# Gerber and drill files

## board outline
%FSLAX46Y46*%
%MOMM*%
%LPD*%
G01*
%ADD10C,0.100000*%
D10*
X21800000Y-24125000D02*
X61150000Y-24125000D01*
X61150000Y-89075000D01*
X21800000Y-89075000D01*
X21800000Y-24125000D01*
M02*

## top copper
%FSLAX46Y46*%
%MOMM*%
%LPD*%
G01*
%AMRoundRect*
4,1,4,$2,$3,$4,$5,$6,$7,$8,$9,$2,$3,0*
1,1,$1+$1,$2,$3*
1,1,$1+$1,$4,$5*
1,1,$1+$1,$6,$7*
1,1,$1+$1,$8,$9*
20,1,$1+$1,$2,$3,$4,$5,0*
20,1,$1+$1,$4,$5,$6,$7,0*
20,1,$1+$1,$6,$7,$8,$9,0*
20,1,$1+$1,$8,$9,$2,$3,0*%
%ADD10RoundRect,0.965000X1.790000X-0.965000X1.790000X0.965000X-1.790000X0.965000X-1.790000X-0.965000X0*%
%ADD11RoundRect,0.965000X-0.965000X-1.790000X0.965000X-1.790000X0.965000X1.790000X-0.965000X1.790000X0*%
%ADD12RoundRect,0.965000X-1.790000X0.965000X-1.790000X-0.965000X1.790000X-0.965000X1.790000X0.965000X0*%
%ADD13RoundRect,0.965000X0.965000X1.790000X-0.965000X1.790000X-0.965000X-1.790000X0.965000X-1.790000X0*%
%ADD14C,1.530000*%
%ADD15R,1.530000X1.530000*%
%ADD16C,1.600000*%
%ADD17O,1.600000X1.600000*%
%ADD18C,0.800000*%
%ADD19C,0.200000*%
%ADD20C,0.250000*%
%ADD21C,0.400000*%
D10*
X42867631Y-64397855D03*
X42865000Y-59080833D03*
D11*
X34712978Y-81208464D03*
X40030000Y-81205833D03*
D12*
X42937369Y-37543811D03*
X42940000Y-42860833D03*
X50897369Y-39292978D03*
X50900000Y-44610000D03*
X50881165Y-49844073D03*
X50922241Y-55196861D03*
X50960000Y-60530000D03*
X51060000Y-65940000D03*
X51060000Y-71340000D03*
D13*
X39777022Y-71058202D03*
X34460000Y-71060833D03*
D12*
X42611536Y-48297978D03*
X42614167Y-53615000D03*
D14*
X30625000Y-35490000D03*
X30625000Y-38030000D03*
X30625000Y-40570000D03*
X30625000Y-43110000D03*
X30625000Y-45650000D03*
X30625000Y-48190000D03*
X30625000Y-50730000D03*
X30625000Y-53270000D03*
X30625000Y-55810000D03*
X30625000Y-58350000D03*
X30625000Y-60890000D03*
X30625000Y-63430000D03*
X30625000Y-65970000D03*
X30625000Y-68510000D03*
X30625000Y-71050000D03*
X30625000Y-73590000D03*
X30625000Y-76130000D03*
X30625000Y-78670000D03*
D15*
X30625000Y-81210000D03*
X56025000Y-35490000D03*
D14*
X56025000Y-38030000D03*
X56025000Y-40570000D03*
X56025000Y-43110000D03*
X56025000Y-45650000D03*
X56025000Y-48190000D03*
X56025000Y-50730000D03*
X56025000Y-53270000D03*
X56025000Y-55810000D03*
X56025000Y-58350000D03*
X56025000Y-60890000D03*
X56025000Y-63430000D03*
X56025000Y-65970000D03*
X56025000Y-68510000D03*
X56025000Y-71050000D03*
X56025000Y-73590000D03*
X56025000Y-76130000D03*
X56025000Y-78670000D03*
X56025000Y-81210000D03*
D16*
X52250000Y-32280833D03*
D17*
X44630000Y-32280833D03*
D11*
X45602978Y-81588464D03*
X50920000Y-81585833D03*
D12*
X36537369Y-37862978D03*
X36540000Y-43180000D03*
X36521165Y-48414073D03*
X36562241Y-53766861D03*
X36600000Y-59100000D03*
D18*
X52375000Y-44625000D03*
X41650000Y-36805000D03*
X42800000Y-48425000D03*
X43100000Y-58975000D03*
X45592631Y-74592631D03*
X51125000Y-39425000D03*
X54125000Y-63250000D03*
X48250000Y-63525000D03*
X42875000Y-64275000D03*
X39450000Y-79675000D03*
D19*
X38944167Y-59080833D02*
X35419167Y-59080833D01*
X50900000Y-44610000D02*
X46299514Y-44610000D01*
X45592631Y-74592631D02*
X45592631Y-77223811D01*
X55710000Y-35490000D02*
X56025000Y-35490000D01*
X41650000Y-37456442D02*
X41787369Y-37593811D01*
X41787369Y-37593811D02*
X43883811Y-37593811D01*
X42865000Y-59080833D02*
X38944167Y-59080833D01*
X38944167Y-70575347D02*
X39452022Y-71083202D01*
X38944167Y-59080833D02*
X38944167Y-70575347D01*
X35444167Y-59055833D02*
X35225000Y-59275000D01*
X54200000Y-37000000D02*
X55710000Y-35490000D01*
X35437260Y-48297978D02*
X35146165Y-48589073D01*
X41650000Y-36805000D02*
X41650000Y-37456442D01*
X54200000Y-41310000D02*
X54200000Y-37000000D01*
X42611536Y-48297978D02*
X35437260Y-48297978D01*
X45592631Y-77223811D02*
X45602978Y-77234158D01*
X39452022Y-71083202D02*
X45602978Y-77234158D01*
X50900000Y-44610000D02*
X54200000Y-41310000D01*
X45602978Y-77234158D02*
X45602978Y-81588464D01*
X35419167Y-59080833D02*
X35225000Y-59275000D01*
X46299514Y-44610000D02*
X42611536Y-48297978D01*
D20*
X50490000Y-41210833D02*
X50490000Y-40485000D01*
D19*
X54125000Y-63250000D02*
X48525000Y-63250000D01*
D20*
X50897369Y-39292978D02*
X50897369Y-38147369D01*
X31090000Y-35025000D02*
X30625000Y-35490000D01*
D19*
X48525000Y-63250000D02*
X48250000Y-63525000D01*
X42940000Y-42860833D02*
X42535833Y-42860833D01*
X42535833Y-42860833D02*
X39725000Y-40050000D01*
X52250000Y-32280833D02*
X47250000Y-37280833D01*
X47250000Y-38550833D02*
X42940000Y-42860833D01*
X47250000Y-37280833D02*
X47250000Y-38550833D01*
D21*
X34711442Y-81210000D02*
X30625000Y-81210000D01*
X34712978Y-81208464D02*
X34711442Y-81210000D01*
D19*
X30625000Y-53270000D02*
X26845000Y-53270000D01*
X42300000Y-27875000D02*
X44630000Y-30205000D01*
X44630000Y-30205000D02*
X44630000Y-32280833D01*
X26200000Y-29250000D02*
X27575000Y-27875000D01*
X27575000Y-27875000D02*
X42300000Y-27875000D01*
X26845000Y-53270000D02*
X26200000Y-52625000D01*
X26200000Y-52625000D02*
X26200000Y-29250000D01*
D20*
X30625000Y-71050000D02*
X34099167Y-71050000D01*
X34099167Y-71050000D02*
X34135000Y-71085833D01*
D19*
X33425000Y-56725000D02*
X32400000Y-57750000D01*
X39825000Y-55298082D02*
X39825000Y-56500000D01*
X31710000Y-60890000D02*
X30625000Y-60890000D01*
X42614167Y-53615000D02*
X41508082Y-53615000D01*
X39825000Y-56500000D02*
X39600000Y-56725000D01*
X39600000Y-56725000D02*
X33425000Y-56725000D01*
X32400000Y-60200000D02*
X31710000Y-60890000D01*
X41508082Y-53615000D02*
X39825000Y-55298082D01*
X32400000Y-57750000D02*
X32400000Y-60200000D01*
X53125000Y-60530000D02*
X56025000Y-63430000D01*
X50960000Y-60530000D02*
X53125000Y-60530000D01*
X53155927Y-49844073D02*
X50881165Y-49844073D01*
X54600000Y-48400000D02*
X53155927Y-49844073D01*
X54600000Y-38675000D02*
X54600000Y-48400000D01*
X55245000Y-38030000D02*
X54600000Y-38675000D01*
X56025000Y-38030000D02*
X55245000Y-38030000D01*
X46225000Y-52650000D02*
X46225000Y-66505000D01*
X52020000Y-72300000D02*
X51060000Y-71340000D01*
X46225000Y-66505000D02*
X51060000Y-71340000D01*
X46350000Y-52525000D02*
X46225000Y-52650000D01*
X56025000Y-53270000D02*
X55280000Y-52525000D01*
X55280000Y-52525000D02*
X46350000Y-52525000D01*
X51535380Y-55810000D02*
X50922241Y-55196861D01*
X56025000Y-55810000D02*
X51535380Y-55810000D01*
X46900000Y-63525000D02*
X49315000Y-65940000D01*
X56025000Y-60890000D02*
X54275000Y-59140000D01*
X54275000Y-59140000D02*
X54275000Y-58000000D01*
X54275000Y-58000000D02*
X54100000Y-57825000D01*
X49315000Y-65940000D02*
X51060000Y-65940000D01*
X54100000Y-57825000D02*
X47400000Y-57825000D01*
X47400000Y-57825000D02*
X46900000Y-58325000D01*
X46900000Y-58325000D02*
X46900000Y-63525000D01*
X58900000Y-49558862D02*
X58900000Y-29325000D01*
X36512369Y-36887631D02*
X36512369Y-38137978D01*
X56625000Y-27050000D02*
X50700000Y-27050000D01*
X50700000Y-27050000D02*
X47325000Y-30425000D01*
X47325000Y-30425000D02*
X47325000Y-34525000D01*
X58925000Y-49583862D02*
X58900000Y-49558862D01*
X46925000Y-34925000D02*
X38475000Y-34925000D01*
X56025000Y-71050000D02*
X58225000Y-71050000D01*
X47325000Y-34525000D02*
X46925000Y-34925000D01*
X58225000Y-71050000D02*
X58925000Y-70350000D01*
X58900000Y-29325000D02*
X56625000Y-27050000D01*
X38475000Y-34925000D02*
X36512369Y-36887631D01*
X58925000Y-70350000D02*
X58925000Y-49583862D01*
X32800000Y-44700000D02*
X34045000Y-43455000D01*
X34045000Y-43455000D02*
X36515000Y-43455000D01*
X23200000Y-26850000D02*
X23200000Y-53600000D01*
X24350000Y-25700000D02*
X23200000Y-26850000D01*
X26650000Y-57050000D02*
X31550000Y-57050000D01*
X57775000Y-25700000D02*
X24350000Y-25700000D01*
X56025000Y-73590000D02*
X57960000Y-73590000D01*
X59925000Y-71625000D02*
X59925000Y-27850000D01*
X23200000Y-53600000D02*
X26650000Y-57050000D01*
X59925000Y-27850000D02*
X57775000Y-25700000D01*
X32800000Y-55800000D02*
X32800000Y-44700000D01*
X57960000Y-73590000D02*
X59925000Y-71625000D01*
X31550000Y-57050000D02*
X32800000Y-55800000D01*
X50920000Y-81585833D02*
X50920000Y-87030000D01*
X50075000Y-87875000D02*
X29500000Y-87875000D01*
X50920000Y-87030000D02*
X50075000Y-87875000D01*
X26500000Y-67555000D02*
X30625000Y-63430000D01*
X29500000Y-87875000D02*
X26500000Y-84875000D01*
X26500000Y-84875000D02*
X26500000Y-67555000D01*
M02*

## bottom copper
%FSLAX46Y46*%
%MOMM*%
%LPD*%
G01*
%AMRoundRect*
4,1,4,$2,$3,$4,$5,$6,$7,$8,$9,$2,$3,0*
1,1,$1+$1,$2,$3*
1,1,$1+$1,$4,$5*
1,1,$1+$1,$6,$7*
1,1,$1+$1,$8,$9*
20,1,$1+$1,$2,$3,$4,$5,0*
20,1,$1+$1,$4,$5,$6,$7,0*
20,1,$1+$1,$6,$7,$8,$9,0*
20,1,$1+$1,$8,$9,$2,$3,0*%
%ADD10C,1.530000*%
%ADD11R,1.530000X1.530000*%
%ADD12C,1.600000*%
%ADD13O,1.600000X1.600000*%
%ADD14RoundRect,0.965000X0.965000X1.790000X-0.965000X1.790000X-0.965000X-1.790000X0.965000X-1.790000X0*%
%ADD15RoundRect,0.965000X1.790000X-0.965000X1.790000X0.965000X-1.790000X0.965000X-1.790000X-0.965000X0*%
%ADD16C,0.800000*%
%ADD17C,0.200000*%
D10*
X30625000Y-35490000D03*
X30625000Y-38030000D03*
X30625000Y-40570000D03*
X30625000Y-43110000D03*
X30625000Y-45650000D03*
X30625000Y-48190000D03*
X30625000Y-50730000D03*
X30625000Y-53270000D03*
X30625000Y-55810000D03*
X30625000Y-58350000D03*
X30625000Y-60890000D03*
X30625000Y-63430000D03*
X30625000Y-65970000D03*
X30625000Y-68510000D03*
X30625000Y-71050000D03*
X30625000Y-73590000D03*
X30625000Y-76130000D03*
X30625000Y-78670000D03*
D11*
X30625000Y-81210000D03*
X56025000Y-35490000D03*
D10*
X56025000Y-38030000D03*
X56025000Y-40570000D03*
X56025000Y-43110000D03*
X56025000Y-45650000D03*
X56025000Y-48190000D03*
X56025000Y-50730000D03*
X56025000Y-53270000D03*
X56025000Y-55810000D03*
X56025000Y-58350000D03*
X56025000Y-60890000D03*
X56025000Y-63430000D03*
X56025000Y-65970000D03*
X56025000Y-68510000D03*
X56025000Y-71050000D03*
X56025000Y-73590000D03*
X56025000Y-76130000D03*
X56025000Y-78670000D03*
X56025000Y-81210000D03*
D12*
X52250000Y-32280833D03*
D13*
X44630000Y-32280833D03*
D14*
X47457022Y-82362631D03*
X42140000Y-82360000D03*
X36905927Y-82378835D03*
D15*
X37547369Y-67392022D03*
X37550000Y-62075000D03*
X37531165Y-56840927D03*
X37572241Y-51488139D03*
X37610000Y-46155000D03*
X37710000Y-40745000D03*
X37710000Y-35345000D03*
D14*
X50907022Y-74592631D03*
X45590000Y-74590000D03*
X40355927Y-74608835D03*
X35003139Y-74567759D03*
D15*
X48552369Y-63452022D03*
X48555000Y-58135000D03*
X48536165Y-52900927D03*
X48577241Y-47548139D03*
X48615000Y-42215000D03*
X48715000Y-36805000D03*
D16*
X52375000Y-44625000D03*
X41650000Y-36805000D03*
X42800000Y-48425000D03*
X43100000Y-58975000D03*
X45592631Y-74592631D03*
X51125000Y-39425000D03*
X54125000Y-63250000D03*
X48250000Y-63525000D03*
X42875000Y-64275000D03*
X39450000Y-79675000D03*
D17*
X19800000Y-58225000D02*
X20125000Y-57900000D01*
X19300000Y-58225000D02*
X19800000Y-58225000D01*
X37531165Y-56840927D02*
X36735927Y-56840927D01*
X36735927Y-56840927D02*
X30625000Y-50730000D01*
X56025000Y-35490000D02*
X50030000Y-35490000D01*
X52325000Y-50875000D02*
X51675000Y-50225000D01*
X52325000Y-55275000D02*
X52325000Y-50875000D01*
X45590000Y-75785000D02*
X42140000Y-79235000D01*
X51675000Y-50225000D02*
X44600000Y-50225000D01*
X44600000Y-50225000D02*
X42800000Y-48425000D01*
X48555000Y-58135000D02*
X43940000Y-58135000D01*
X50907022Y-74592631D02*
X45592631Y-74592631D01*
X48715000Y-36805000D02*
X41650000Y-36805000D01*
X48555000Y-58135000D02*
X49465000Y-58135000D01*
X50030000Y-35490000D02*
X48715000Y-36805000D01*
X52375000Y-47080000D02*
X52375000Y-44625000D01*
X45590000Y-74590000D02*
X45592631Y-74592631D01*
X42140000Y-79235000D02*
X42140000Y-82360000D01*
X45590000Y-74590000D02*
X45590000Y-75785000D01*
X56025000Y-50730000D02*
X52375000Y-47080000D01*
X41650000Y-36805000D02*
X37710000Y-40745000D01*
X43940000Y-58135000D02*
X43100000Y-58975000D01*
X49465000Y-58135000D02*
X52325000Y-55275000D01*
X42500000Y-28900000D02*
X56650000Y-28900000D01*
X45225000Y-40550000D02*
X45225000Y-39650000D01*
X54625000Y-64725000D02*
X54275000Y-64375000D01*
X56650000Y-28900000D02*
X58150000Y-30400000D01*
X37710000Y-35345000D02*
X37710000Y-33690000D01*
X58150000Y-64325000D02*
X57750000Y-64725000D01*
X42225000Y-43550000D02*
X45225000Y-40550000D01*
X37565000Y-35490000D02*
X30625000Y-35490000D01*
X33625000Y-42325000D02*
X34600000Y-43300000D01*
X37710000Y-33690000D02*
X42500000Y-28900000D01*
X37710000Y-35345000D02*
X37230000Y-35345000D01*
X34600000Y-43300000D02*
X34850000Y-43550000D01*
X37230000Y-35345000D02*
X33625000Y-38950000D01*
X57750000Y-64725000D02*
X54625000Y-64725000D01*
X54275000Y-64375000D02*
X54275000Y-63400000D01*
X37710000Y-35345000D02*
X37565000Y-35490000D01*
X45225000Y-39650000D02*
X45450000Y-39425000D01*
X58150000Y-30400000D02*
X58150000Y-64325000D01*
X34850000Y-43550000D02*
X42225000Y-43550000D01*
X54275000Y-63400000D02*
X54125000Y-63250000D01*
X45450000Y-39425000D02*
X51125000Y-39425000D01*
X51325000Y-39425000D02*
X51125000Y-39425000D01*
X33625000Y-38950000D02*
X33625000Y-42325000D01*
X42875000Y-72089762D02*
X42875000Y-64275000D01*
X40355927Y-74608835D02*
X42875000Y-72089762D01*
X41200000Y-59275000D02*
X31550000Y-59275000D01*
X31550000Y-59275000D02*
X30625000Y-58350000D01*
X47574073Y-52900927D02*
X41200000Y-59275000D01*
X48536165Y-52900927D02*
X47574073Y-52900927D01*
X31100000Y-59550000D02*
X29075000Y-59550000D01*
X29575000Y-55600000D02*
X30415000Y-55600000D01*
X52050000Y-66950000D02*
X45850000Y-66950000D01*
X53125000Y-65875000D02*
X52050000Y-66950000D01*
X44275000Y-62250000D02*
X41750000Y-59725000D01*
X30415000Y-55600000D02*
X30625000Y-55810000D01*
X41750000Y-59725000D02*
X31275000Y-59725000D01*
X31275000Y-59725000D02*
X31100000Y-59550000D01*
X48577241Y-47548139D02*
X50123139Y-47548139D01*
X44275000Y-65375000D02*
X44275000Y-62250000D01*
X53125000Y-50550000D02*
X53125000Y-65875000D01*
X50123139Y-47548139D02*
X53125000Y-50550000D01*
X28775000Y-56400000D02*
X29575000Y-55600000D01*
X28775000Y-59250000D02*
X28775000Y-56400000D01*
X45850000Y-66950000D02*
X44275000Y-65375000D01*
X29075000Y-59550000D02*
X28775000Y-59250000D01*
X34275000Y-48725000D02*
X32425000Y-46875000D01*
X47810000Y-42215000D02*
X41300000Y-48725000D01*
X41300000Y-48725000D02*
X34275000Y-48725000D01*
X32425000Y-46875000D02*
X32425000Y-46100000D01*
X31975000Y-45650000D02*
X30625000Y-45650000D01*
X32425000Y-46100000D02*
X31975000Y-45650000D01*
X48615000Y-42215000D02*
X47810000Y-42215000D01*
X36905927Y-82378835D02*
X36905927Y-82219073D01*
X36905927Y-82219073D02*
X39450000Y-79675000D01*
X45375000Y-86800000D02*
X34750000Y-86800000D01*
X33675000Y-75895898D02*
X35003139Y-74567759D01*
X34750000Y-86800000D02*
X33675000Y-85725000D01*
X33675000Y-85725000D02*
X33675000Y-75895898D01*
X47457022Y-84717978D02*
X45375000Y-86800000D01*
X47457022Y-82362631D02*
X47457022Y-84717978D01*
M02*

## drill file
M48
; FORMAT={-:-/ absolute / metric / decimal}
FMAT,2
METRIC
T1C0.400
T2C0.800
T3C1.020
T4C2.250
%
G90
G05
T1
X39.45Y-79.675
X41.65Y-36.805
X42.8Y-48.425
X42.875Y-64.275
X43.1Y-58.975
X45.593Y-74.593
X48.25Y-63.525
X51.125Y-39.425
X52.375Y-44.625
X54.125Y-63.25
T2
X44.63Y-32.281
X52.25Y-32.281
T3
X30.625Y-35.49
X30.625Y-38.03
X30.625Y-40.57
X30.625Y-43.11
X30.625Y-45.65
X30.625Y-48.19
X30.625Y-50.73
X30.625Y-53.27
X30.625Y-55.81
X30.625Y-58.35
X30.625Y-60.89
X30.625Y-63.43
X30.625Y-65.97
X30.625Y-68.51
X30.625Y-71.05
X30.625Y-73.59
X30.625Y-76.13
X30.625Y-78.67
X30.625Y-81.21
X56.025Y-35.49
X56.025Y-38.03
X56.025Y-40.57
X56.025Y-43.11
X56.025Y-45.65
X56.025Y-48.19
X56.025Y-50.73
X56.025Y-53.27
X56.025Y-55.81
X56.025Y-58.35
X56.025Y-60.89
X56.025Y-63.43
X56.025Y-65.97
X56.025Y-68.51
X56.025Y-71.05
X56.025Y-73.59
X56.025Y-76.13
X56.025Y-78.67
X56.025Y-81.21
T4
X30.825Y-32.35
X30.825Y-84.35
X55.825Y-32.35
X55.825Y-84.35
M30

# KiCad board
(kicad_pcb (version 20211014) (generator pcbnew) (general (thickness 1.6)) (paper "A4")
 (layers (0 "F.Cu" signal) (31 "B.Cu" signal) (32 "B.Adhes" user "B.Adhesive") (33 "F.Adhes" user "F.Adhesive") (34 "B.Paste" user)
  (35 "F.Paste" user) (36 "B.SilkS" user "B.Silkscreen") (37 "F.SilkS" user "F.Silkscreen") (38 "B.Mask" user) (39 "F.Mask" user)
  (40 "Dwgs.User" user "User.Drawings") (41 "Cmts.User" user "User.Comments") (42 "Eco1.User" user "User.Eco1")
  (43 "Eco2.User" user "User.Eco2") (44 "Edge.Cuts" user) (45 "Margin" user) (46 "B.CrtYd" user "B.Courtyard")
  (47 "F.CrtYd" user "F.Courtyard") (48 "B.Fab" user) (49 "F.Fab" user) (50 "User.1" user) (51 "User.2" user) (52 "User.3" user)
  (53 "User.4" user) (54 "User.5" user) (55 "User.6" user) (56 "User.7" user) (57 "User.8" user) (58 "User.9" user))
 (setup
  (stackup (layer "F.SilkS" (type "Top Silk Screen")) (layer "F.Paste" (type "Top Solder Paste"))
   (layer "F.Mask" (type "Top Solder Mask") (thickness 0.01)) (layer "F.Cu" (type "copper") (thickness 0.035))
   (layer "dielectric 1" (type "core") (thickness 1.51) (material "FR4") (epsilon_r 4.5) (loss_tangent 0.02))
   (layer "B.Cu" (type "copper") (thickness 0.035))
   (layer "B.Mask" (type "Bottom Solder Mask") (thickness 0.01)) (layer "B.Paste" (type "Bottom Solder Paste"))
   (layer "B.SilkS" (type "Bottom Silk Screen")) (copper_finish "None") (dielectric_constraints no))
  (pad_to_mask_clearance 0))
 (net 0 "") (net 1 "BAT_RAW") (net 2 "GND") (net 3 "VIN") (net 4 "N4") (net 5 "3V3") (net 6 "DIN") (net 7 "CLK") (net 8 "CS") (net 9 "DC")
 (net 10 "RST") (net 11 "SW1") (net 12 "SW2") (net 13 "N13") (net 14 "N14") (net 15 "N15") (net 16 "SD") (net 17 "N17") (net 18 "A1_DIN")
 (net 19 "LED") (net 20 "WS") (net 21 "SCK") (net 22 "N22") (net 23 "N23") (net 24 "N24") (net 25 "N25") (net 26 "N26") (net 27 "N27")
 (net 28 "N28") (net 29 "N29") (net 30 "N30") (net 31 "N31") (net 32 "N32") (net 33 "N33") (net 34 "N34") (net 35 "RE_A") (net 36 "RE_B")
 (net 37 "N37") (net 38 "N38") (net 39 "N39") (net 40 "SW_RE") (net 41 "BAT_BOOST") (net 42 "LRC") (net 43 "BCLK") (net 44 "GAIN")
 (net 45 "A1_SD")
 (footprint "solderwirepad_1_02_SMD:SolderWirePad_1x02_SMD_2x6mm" (layer "F.Cu") (at 43.89 61.680833 90)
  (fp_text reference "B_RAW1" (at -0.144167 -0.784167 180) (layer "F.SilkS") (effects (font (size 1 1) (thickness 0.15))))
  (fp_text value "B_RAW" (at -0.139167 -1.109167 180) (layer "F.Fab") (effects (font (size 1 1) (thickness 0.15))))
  (pad "1" smd roundrect (at -2.717022 -1.022369 90) (size 3.86 5.51) (layers "F.Cu" "F.Paste" "F.Mask") (roundrect_rratio 0.25)
   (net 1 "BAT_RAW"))
  (pad "2" smd roundrect (at 2.6 -1.025 90) (size 3.86 5.51) (layers "F.Cu" "F.Paste" "F.Mask") (roundrect_rratio 0.25) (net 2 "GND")))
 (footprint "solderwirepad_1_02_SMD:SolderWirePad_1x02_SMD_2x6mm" (layer "F.Cu") (at 37.43 82.230833)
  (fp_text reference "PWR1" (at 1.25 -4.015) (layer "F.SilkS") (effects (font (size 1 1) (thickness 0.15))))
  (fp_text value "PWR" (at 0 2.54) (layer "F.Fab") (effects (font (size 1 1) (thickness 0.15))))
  (pad "1" smd roundrect (at -2.717022 -1.022369) (size 3.86 5.51) (layers "F.Cu" "F.Paste" "F.Mask") (roundrect_rratio 0.25) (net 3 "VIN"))
  (pad "2" smd roundrect (at 2.6 -1.025) (size 3.86 5.51) (layers "F.Cu" "F.Paste" "F.Mask") (roundrect_rratio 0.25) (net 3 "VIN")))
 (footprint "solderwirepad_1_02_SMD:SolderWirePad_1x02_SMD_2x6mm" (layer "F.Cu") (at 41.915 40.260833 -90)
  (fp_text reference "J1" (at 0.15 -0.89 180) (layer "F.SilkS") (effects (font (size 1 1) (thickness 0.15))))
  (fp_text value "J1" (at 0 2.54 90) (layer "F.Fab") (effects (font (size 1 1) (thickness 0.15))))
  (pad "1" smd roundrect (at -2.717022 -1.022369 270) (size 3.86 5.51) (layers "F.Cu" "F.Paste" "F.Mask") (roundrect_rratio 0.25)
   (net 2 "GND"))
  (pad "2" smd roundrect (at 2.6 -1.025 270) (size 3.86 5.51) (layers "F.Cu" "F.Paste" "F.Mask") (roundrect_rratio 0.25) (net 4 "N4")))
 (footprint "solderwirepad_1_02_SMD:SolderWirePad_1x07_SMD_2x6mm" (layer "F.Cu") (at 49.875 54.51 -90)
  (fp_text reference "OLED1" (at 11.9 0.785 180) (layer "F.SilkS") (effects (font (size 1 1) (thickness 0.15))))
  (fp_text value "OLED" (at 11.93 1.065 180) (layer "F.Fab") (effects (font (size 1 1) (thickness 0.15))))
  (pad "1" smd roundrect (at -15.217022 -1.022369 270) (size 3.86 5.51) (layers "F.Cu" "F.Paste" "F.Mask") (roundrect_rratio 0.25)
   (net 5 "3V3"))
  (pad "2" smd roundrect (at -9.9 -1.025 270) (size 3.86 5.51) (layers "F.Cu" "F.Paste" "F.Mask") (roundrect_rratio 0.25) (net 2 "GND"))
  (pad "3" smd roundrect (at -4.665927 -1.006165 270) (size 3.86 5.51) (layers "F.Cu" "F.Paste" "F.Mask") (roundrect_rratio 0.25)
   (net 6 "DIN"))
  (pad "4" smd roundrect (at 0.686861 -1.047241 270) (size 3.86 5.51) (layers "F.Cu" "F.Paste" "F.Mask") (roundrect_rratio 0.25)
   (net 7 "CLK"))
  (pad "5" smd roundrect (at 6.02 -1.085 270) (size 3.86 5.51) (layers "F.Cu" "F.Paste" "F.Mask") (roundrect_rratio 0.25) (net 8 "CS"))
  (pad "6" smd roundrect (at 11.43 -1.185 270) (size 3.86 5.51) (layers "F.Cu" "F.Paste" "F.Mask") (roundrect_rratio 0.25) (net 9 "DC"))
  (pad "7" smd roundrect (at 16.83 -1.185 270) (size 3.86 5.51) (layers "F.Cu" "F.Paste" "F.Mask") (roundrect_rratio 0.25) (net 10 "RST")))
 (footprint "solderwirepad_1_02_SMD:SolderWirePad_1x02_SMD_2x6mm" (layer "F.Cu") (at 37.06 70.035833 180)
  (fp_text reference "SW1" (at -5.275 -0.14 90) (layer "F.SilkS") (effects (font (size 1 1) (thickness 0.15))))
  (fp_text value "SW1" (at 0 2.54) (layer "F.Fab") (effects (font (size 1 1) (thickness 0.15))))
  (pad "1" smd roundrect (at -2.717022 -1.022369 180) (size 3.86 5.51) (layers "F.Cu" "F.Paste" "F.Mask") (roundrect_rratio 0.25)
   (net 2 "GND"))
  (pad "2" smd roundrect (at 2.6 -1.025 180) (size 3.86 5.51) (layers "F.Cu" "F.Paste" "F.Mask") (roundrect_rratio 0.25) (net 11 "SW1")))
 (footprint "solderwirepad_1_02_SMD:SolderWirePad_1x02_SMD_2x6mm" (layer "F.Cu") (at 41.589167 51.015 -90)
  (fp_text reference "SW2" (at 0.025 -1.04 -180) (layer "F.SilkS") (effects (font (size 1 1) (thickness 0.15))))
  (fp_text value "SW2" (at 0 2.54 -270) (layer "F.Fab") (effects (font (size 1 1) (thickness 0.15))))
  (pad "1" smd roundrect (at -2.717022 -1.022369 270) (size 3.86 5.51) (layers "F.Cu" "F.Paste" "F.Mask") (roundrect_rratio 0.25)
   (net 2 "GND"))
  (pad "2" smd roundrect (at 2.6 -1.025 270) (size 3.86 5.51) (layers "F.Cu" "F.Paste" "F.Mask") (roundrect_rratio 0.25) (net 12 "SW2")))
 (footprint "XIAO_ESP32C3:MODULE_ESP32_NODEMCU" (layer "F.Cu") (at 43.325 58.35)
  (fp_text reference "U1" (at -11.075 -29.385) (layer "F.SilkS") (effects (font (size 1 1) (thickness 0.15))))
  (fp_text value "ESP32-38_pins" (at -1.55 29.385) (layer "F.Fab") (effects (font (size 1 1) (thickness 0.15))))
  (pad "" np_thru_hole circle (at -12.5 26) (size 2.25 2.25) (drill 2.25) (layers *.Cu *.Mask))
  (pad "" np_thru_hole circle (at 12.5 26) (size 2.25 2.25) (drill 2.25) (layers *.Cu *.Mask))
  (pad "" np_thru_hole circle (at 12.5 -26) (size 2.25 2.25) (drill 2.25) (layers *.Cu *.Mask))
  (pad "" np_thru_hole circle (at -12.5 -26) (size 2.25 2.25) (drill 2.25) (layers *.Cu *.Mask))
  (pad "J1_1" thru_hole circle (at -12.7 -22.86) (size 1.53 1.53) (drill 1.02) (layers *.Cu *.Mask) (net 5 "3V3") (solder_mask_margin 0.102))
  (pad "J1_2" thru_hole circle (at -12.7 -20.32 90) (size 1.53 1.53) (drill 1.02) (layers *.Cu *.Mask) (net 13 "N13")
   (solder_mask_margin 0.102))
  (pad "J1_3" thru_hole circle (at -12.7 -17.78) (size 1.53 1.53) (drill 1.02) (layers *.Cu *.Mask) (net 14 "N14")
   (solder_mask_margin 0.102))
  (pad "J1_4" thru_hole circle (at -12.7 -15.24) (size 1.53 1.53) (drill 1.02) (layers *.Cu *.Mask) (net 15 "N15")
   (solder_mask_margin 0.102))
  (pad "J1_5" thru_hole circle (at -12.7 -12.7) (size 1.53 1.53) (drill 1.02) (layers *.Cu *.Mask) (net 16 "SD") (solder_mask_margin 0.102))
  (pad "J1_6" thru_hole circle (at -12.7 -10.16) (size 1.53 1.53) (drill 1.02) (layers *.Cu *.Mask) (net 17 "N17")
   (solder_mask_margin 0.102))
  (pad "J1_7" thru_hole circle (at -12.7 -7.62) (size 1.53 1.53) (drill 1.02) (layers *.Cu *.Mask) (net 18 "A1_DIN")
   (solder_mask_margin 0.102))
  (pad "J1_8" thru_hole circle (at -12.7 -5.08) (size 1.53 1.53) (drill 1.02) (layers *.Cu *.Mask) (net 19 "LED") (solder_mask_margin 0.102))
  (pad "J1_9" thru_hole circle (at -12.7 -2.54) (size 1.53 1.53) (drill 1.02) (layers *.Cu *.Mask) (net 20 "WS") (solder_mask_margin 0.102))
  (pad "J1_10" thru_hole circle (at -12.7 0) (size 1.53 1.53) (drill 1.02) (layers *.Cu *.Mask) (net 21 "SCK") (solder_mask_margin 0.102))
  (pad "J1_11" thru_hole circle (at -12.7 2.54) (size 1.53 1.53) (drill 1.02) (layers *.Cu *.Mask) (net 12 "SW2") (solder_mask_margin 0.102))
  (pad "J1_12" thru_hole circle (at -12.7 5.08) (size 1.53 1.53) (drill 1.02) (layers *.Cu *.Mask) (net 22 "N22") (solder_mask_margin 0.102))
  (pad "J1_13" thru_hole circle (at -12.7 7.62) (size 1.53 1.53) (drill 1.02) (layers *.Cu *.Mask) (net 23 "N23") (solder_mask_margin 0.102))
  (pad "J1_14" thru_hole circle (at -12.7 10.16) (size 1.53 1.53) (drill 1.02) (layers *.Cu *.Mask) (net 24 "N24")
   (solder_mask_margin 0.102))
  (pad "J1_15" thru_hole circle (at -12.7 12.7) (size 1.53 1.53) (drill 1.02) (layers *.Cu *.Mask) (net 11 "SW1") (solder_mask_margin 0.102))
  (pad "J1_16" thru_hole circle (at -12.7 15.24) (size 1.53 1.53) (drill 1.02) (layers *.Cu *.Mask) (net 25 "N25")
   (solder_mask_margin 0.102))
  (pad "J1_17" thru_hole circle (at -12.7 17.78) (size 1.53 1.53) (drill 1.02) (layers *.Cu *.Mask) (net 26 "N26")
   (solder_mask_margin 0.102))
  (pad "J1_18" thru_hole circle (at -12.7 20.32) (size 1.53 1.53) (drill 1.02) (layers *.Cu *.Mask) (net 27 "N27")
   (solder_mask_margin 0.102))
  (pad "J1_19" thru_hole rect (at -12.7 22.86) (size 1.53 1.53) (drill 1.02) (layers *.Cu *.Mask) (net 3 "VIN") (solder_mask_margin 0.102))
  (pad "J2_1" thru_hole rect (at 12.7 -22.86) (size 1.53 1.53) (drill 1.02) (layers *.Cu *.Mask) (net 2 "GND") (solder_mask_margin 0.102))
  (pad "J2_2" thru_hole circle (at 12.7 -20.32) (size 1.53 1.53) (drill 1.02) (layers *.Cu *.Mask) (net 6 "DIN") (solder_mask_margin 0.102))
  (pad "J2_3" thru_hole circle (at 12.7 -17.78) (size 1.53 1.53) (drill 1.02) (layers *.Cu *.Mask) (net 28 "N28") (solder_mask_margin 0.102))
  (pad "J2_4" thru_hole circle (at 12.7 -15.24) (size 1.53 1.53) (drill 1.02) (layers *.Cu *.Mask) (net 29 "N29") (solder_mask_margin 0.102))
  (pad "J2_5" thru_hole circle (at 12.7 -12.7) (size 1.53 1.53) (drill 1.02) (layers *.Cu *.Mask) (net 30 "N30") (solder_mask_margin 0.102))
  (pad "J2_6" thru_hole circle (at 12.7 -10.16) (size 1.53 1.53) (drill 1.02) (layers *.Cu *.Mask) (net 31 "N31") (solder_mask_margin 0.102))
  (pad "J2_7" thru_hole circle (at 12.7 -7.62) (size 1.53 1.53) (drill 1.02) (layers *.Cu *.Mask) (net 2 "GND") (solder_mask_margin 0.102))
  (pad "J2_8" thru_hole circle (at 12.7 -5.08) (size 1.53 1.53) (drill 1.02) (layers *.Cu *.Mask) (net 10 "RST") (solder_mask_margin 0.102))
  (pad "J2_9" thru_hole circle (at 12.7 -2.54) (size 1.53 1.53) (drill 1.02) (layers *.Cu *.Mask) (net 7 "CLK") (solder_mask_margin 0.102))
  (pad "J2_10" thru_hole circle (at 12.7 0) (size 1.53 1.53) (drill 1.02) (layers *.Cu *.Mask) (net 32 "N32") (solder_mask_margin 0.102))
  (pad "J2_11" thru_hole circle (at 12.7 2.54) (size 1.53 1.53) (drill 1.02) (layers *.Cu *.Mask) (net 9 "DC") (solder_mask_margin 0.102))
  (pad "J2_12" thru_hole circle (at 12.7 5.08) (size 1.53 1.53) (drill 1.02) (layers *.Cu *.Mask) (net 8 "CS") (solder_mask_margin 0.102))
  (pad "J2_13" thru_hole circle (at 12.7 7.62) (size 1.53 1.53) (drill 1.02) (layers *.Cu *.Mask) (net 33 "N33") (solder_mask_margin 0.102))
  (pad "J2_14" thru_hole circle (at 12.7 10.16) (size 1.53 1.53) (drill 1.02) (layers *.Cu *.Mask) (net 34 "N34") (solder_mask_margin 0.102))
  (pad "J2_15" thru_hole circle (at 12.7 12.7) (size 1.53 1.53) (drill 1.02) (layers *.Cu *.Mask) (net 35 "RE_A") (solder_mask_margin 0.102))
  (pad "J2_16" thru_hole circle (at 12.7 15.24) (size 1.53 1.53) (drill 1.02) (layers *.Cu *.Mask) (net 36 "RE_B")
   (solder_mask_margin 0.102))
  (pad "J2_17" thru_hole circle (at 12.7 17.78) (size 1.53 1.53) (drill 1.02) (layers *.Cu *.Mask) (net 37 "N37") (solder_mask_margin 0.102))
  (pad "J2_18" thru_hole circle (at 12.7 20.32) (size 1.53 1.53) (drill 1.02) (layers *.Cu *.Mask) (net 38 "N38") (solder_mask_margin 0.102))
  (pad "J2_19" thru_hole circle (at 12.7 22.86) (size 1.53 1.53) (drill 1.02) (layers *.Cu *.Mask) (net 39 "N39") (solder_mask_margin 0.102)))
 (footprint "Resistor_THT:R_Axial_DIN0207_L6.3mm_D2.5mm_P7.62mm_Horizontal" (layer "F.Cu") (at 52.25 32.280833 180)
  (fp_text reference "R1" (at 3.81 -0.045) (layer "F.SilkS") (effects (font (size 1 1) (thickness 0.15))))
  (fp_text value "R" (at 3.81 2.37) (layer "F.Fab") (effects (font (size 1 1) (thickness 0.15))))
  (pad "1" thru_hole circle (at 0 0 180) (size 1.6 1.6) (drill 0.8) (layers *.Cu *.Mask) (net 4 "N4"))
  (pad "2" thru_hole oval (at 7.62 0 180) (size 1.6 1.6) (drill 0.8) (layers *.Cu *.Mask) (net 19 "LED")))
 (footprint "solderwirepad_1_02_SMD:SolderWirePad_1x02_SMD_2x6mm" (layer "F.Cu") (at 48.32 82.610833)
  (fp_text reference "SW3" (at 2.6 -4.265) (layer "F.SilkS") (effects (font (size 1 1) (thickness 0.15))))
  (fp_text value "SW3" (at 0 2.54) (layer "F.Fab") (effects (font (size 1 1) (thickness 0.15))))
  (pad "1" smd roundrect (at -2.717022 -1.022369) (size 3.86 5.51) (layers "F.Cu" "F.Paste" "F.Mask") (roundrect_rratio 0.25) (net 2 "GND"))
  (pad "2" smd roundrect (at 2.6 -1.025) (size 3.86 5.51) (layers "F.Cu" "F.Paste" "F.Mask") (roundrect_rratio 0.25) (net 22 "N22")))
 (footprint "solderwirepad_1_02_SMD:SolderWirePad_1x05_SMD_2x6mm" (layer "F.Cu") (at 35.515 43.08 -90)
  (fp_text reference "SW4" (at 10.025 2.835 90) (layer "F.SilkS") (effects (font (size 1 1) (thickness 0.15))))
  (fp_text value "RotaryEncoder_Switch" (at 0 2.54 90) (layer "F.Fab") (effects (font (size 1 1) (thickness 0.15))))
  (pad "1" smd roundrect (at -5.217022 -1.022369 270) (size 3.86 5.51) (layers "F.Cu" "F.Paste" "F.Mask") (roundrect_rratio 0.25)
   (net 35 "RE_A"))
  (pad "2" smd roundrect (at 0.1 -1.025 270) (size 3.86 5.51) (layers "F.Cu" "F.Paste" "F.Mask") (roundrect_rratio 0.25) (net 36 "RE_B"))
  (pad "3" smd roundrect (at 5.334073 -1.006165 270) (size 3.86 5.51) (layers "F.Cu" "F.Paste" "F.Mask") (roundrect_rratio 0.25)
   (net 2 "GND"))
  (pad "4" smd roundrect (at 10.686861 -1.047241 270) (size 3.86 5.51) (layers "F.Cu" "F.Paste" "F.Mask") (roundrect_rratio 0.25)
   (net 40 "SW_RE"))
  (pad "5" smd roundrect (at 16.02 -1.085 270) (size 3.86 5.51) (layers "F.Cu" "F.Paste" "F.Mask") (roundrect_rratio 0.25) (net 2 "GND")))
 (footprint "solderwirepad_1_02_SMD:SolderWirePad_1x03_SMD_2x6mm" (layer "B.Cu") (at 42.24 83.385 180)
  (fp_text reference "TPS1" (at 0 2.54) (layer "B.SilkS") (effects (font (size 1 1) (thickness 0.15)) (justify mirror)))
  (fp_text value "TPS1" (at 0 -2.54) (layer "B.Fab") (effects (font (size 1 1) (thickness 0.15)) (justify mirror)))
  (pad "1" smd roundrect (at -5.217022 1.022369 180) (size 3.86 5.51) (layers "B.Cu" "B.Paste" "B.Mask") (roundrect_rratio 0.25)
   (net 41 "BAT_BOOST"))
  (pad "2" smd roundrect (at 0.1 1.025 180) (size 3.86 5.51) (layers "B.Cu" "B.Paste" "B.Mask") (roundrect_rratio 0.25) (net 2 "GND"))
  (pad "3" smd roundrect (at 5.334073 1.006165 180) (size 3.86 5.51) (layers "B.Cu" "B.Paste" "B.Mask") (roundrect_rratio 0.25)
   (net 3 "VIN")))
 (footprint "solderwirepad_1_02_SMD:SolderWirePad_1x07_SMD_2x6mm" (layer "B.Cu") (at 36.525 52.175 90)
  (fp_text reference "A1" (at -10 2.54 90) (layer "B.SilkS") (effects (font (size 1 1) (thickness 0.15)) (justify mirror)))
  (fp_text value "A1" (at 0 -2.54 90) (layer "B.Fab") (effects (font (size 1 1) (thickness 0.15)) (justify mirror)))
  (pad "1" smd roundrect (at -15.217022 1.022369 90) (size 3.86 5.51) (layers "B.Cu" "B.Paste" "B.Mask") (roundrect_rratio 0.25)
   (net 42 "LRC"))
  (pad "2" smd roundrect (at -9.9 1.025 90) (size 3.86 5.51) (layers "B.Cu" "B.Paste" "B.Mask") (roundrect_rratio 0.25) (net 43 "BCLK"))
  (pad "3" smd roundrect (at -4.665927 1.006165 90) (size 3.86 5.51) (layers "B.Cu" "B.Paste" "B.Mask") (roundrect_rratio 0.25)
   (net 18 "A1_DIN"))
  (pad "4" smd roundrect (at 0.686861 1.047241 90) (size 3.86 5.51) (layers "B.Cu" "B.Paste" "B.Mask") (roundrect_rratio 0.25)
   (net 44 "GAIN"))
  (pad "5" smd roundrect (at 6.02 1.085 90) (size 3.86 5.51) (layers "B.Cu" "B.Paste" "B.Mask") (roundrect_rratio 0.25) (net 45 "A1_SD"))
  (pad "6" smd roundrect (at 11.43 1.185 90) (size 3.86 5.51) (layers "B.Cu" "B.Paste" "B.Mask") (roundrect_rratio 0.25) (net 2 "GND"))
  (pad "7" smd roundrect (at 16.83 1.185 90) (size 3.86 5.51) (layers "B.Cu" "B.Paste" "B.Mask") (roundrect_rratio 0.25) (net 5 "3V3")))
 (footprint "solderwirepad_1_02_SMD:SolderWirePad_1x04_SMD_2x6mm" (layer "B.Cu") (at 42.69 75.615 180)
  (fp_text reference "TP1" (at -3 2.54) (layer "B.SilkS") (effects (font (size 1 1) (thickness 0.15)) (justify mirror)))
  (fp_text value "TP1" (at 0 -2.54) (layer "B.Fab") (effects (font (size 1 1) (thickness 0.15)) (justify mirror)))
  (pad "1" smd roundrect (at -8.217022 1.022369 180) (size 3.86 5.51) (layers "B.Cu" "B.Paste" "B.Mask") (roundrect_rratio 0.25)
   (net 2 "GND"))
  (pad "2" smd roundrect (at -2.9 1.025 180) (size 3.86 5.51) (layers "B.Cu" "B.Paste" "B.Mask") (roundrect_rratio 0.25) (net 2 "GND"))
  (pad "3" smd roundrect (at 2.334073 1.006165 180) (size 3.86 5.51) (layers "B.Cu" "B.Paste" "B.Mask") (roundrect_rratio 0.25)
   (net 1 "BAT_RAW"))
  (pad "4" smd roundrect (at 7.686861 1.047241 180) (size 3.86 5.51) (layers "B.Cu" "B.Paste" "B.Mask") (roundrect_rratio 0.25)
   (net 41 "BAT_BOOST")))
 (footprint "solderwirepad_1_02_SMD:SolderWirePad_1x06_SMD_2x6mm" (layer "B.Cu") (at 47.53 48.235 90)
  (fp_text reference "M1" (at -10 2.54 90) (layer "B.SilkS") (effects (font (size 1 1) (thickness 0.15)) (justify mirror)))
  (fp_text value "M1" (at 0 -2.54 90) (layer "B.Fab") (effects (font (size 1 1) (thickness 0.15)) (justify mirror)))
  (pad "1" smd roundrect (at -15.217022 1.022369 90) (size 3.86 5.51) (layers "B.Cu" "B.Paste" "B.Mask") (roundrect_rratio 0.25)
   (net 5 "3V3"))
  (pad "2" smd roundrect (at -9.9 1.025 90) (size 3.86 5.51) (layers "B.Cu" "B.Paste" "B.Mask") (roundrect_rratio 0.25) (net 2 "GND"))
  (pad "3" smd roundrect (at -4.665927 1.006165 90) (size 3.86 5.51) (layers "B.Cu" "B.Paste" "B.Mask") (roundrect_rratio 0.25)
   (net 21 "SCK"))
  (pad "4" smd roundrect (at 0.686861 1.047241 90) (size 3.86 5.51) (layers "B.Cu" "B.Paste" "B.Mask") (roundrect_rratio 0.25) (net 20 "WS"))
  (pad "5" smd roundrect (at 6.02 1.085 90) (size 3.86 5.51) (layers "B.Cu" "B.Paste" "B.Mask") (roundrect_rratio 0.25) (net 16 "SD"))
  (pad "6" smd roundrect (at 11.43 1.185 90) (size 3.86 5.51) (layers "B.Cu" "B.Paste" "B.Mask") (roundrect_rratio 0.25) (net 2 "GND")))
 (gr_rect (start 21.8 24.125) (end 61.15 89.075) (layer "Edge.Cuts") (width 0.1) (fill none))
 (segment (start 19.8 58.225) (end 20.125 57.9) (width 0.2) (layer "B.Cu") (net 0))
 (segment (start 19.3 58.225) (end 19.8 58.225) (width 0.2) (layer "B.Cu") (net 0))
 (segment (start 37.531165 56.840927) (end 36.735927 56.840927) (width 0.2) (layer "B.Cu") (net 18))
 (segment (start 36.735927 56.840927) (end 30.625 50.73) (width 0.2) (layer "B.Cu") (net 18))
 (segment (start 38.944167 59.080833) (end 35.419167 59.080833) (width 0.2) (layer "F.Cu") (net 2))
 (segment (start 50.9 44.61) (end 46.299514 44.61) (width 0.2) (layer "F.Cu") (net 2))
 (segment (start 45.592631 74.592631) (end 45.592631 77.223811) (width 0.2) (layer "F.Cu") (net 2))
 (segment (start 55.71 35.49) (end 56.025 35.49) (width 0.2) (layer "F.Cu") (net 2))
 (segment (start 41.65 37.456442) (end 41.787369 37.593811) (width 0.2) (layer "F.Cu") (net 2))
 (segment (start 41.787369 37.593811) (end 43.883811 37.593811) (width 0.2) (layer "F.Cu") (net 2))
 (segment (start 42.865 59.080833) (end 38.944167 59.080833) (width 0.2) (layer "F.Cu") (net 2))
 (segment (start 38.944167 70.575347) (end 39.452022 71.083202) (width 0.2) (layer "F.Cu") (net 2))
 (segment (start 38.944167 59.080833) (end 38.944167 70.575347) (width 0.2) (layer "F.Cu") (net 2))
 (segment (start 35.444167 59.055833) (end 35.225 59.275) (width 0.2) (layer "F.Cu") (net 2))
 (segment (start 54.2 37) (end 55.71 35.49) (width 0.2) (layer "F.Cu") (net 2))
 (segment (start 35.43726 48.297978) (end 35.146165 48.589073) (width 0.2) (layer "F.Cu") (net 2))
 (segment (start 41.65 36.805) (end 41.65 37.456442) (width 0.2) (layer "F.Cu") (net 2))
 (segment (start 54.2 41.31) (end 54.2 37) (width 0.2) (layer "F.Cu") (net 2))
 (segment (start 42.611536 48.297978) (end 35.43726 48.297978) (width 0.2) (layer "F.Cu") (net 2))
 (segment (start 45.592631 77.223811) (end 45.602978 77.234158) (width 0.2) (layer "F.Cu") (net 2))
 (segment (start 39.452022 71.083202) (end 45.602978 77.234158) (width 0.2) (layer "F.Cu") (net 2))
 (segment (start 50.9 44.61) (end 54.2 41.31) (width 0.2) (layer "F.Cu") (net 2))
 (segment (start 45.602978 77.234158) (end 45.602978 81.588464) (width 0.2) (layer "F.Cu") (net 2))
 (segment (start 35.419167 59.080833) (end 35.225 59.275) (width 0.2) (layer "F.Cu") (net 2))
 (segment (start 46.299514 44.61) (end 42.611536 48.297978) (width 0.2) (layer "F.Cu") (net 2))
 (via (at 52.375 44.625) (size 0.8) (drill 0.4) (layers "F.Cu" "B.Cu") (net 2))
 (via (at 41.65 36.805) (size 0.8) (drill 0.4) (layers "F.Cu" "B.Cu") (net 2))
 (via (at 42.8 48.425) (size 0.8) (drill 0.4) (layers "F.Cu" "B.Cu") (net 2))
 (via (at 43.1 58.975) (size 0.8) (drill 0.4) (layers "F.Cu" "B.Cu") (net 2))
 (via (at 45.592631 74.592631) (size 0.8) (drill 0.4) (layers "F.Cu" "B.Cu") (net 2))
 (segment (start 56.025 35.49) (end 50.03 35.49) (width 0.2) (layer "B.Cu") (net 2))
 (segment (start 52.325 50.875) (end 51.675 50.225) (width 0.2) (layer "B.Cu") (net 2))
 (segment (start 52.325 55.275) (end 52.325 50.875) (width 0.2) (layer "B.Cu") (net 2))
 (segment (start 45.59 75.785) (end 42.14 79.235) (width 0.2) (layer "B.Cu") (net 2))
 (segment (start 51.675 50.225) (end 44.6 50.225) (width 0.2) (layer "B.Cu") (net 2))
 (segment (start 44.6 50.225) (end 42.8 48.425) (width 0.2) (layer "B.Cu") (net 2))
 (segment (start 48.555 58.135) (end 43.94 58.135) (width 0.2) (layer "B.Cu") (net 2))
 (segment (start 50.907022 74.592631) (end 45.592631 74.592631) (width 0.2) (layer "B.Cu") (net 2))
 (segment (start 48.715 36.805) (end 41.65 36.805) (width 0.2) (layer "B.Cu") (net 2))
 (segment (start 48.555 58.135) (end 49.465 58.135) (width 0.2) (layer "B.Cu") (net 2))
 (segment (start 50.03 35.49) (end 48.715 36.805) (width 0.2) (layer "B.Cu") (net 2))
 (segment (start 52.375 47.08) (end 52.375 44.625) (width 0.2) (layer "B.Cu") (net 2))
 (segment (start 45.59 74.59) (end 45.592631 74.592631) (width 0.2) (layer "B.Cu") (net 2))
 (segment (start 42.14 79.235) (end 42.14 82.36) (width 0.2) (layer "B.Cu") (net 2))
 (segment (start 45.59 74.59) (end 45.59 75.785) (width 0.2) (layer "B.Cu") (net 2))
 (segment (start 56.025 50.73) (end 52.375 47.08) (width 0.2) (layer "B.Cu") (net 2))
 (segment (start 41.65 36.805) (end 37.71 40.745) (width 0.2) (layer "B.Cu") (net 2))
 (segment (start 43.94 58.135) (end 43.1 58.975) (width 0.2) (layer "B.Cu") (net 2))
 (segment (start 49.465 58.135) (end 52.325 55.275) (width 0.2) (layer "B.Cu") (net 2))
 (segment (start 50.49 41.210833) (end 50.49 40.485) (width 0.25) (layer "F.Cu") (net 5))
 (segment (start 54.125 63.25) (end 48.525 63.25) (width 0.2) (layer "F.Cu") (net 5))
 (segment (start 50.897369 39.292978) (end 50.897369 38.147369) (width 0.25) (layer "F.Cu") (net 5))
 (segment (start 31.09 35.025) (end 30.625 35.49) (width 0.25) (layer "F.Cu") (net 5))
 (segment (start 48.525 63.25) (end 48.25 63.525) (width 0.2) (layer "F.Cu") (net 5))
 (via (at 51.125 39.425) (size 0.8) (drill 0.4) (layers "F.Cu" "B.Cu") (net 5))
 (via (at 54.125 63.25) (size 0.8) (drill 0.4) (layers "F.Cu" "B.Cu") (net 5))
 (via (at 48.25 63.525) (size 0.8) (drill 0.4) (layers "F.Cu" "B.Cu") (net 5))
 (segment (start 42.5 28.9) (end 56.65 28.9) (width 0.2) (layer "B.Cu") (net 5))
 (segment (start 45.225 40.55) (end 45.225 39.65) (width 0.2) (layer "B.Cu") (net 5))
 (segment (start 54.625 64.725) (end 54.275 64.375) (width 0.2) (layer "B.Cu") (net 5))
 (segment (start 56.65 28.9) (end 58.15 30.4) (width 0.2) (layer "B.Cu") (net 5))
 (segment (start 37.71 35.345) (end 37.71 33.69) (width 0.2) (layer "B.Cu") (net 5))
 (segment (start 58.15 64.325) (end 57.75 64.725) (width 0.2) (layer "B.Cu") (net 5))
 (segment (start 42.225 43.55) (end 45.225 40.55) (width 0.2) (layer "B.Cu") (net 5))
 (segment (start 37.565 35.49) (end 30.625 35.49) (width 0.2) (layer "B.Cu") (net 5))
 (segment (start 33.625 42.325) (end 34.6 43.3) (width 0.2) (layer "B.Cu") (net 5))
 (segment (start 37.71 33.69) (end 42.5 28.9) (width 0.2) (layer "B.Cu") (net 5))
 (segment (start 37.71 35.345) (end 37.23 35.345) (width 0.2) (layer "B.Cu") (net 5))
 (segment (start 34.6 43.3) (end 34.85 43.55) (width 0.2) (layer "B.Cu") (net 5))
 (segment (start 37.23 35.345) (end 33.625 38.95) (width 0.2) (layer "B.Cu") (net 5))
 (segment (start 57.75 64.725) (end 54.625 64.725) (width 0.2) (layer "B.Cu") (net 5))
 (segment (start 54.275 64.375) (end 54.275 63.4) (width 0.2) (layer "B.Cu") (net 5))
 (segment (start 37.71 35.345) (end 37.565 35.49) (width 0.2) (layer "B.Cu") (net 5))
 (segment (start 45.225 39.65) (end 45.45 39.425) (width 0.2) (layer "B.Cu") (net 5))
 (segment (start 58.15 30.4) (end 58.15 64.325) (width 0.2) (layer "B.Cu") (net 5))
 (segment (start 34.85 43.55) (end 42.225 43.55) (width 0.2) (layer "B.Cu") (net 5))
 (segment (start 54.275 63.4) (end 54.125 63.25) (width 0.2) (layer "B.Cu") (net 5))
 (segment (start 45.45 39.425) (end 51.125 39.425) (width 0.2) (layer "B.Cu") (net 5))
 (segment (start 51.325 39.425) (end 51.125 39.425) (width 0.2) (layer "B.Cu") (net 5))
 (segment (start 33.625 38.95) (end 33.625 42.325) (width 0.2) (layer "B.Cu") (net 5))
 (via (at 42.875 64.275) (size 0.8) (drill 0.4) (layers "F.Cu" "B.Cu") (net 1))
 (segment (start 42.875 72.089762) (end 42.875 64.275) (width 0.2) (layer "B.Cu") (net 1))
 (segment (start 40.355927 74.608835) (end 42.875 72.089762) (width 0.2) (layer "B.Cu") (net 1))
 (segment (start 42.94 42.860833) (end 42.535833 42.860833) (width 0.2) (layer "F.Cu") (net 4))
 (segment (start 42.535833 42.860833) (end 39.725 40.05) (width 0.2) (layer "F.Cu") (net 4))
 (segment (start 52.25 32.280833) (end 47.25 37.280833) (width 0.2) (layer "F.Cu") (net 4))
 (segment (start 47.25 38.550833) (end 42.94 42.860833) (width 0.2) (layer "F.Cu") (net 4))
 (segment (start 47.25 37.280833) (end 47.25 38.550833) (width 0.2) (layer "F.Cu") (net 4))
 (segment (start 41.2 59.275) (end 31.55 59.275) (width 0.2) (layer "B.Cu") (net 21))
 (segment (start 31.55 59.275) (end 30.625 58.35) (width 0.2) (layer "B.Cu") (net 21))
 (segment (start 47.574073 52.900927) (end 41.2 59.275) (width 0.2) (layer "B.Cu") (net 21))
 (segment (start 48.536165 52.900927) (end 47.574073 52.900927) (width 0.2) (layer "B.Cu") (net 21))
 (segment (start 31.1 59.55) (end 29.075 59.55) (width 0.2) (layer "B.Cu") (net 20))
 (segment (start 29.575 55.6) (end 30.415 55.6) (width 0.2) (layer "B.Cu") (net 20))
 (segment (start 52.05 66.95) (end 45.85 66.95) (width 0.2) (layer "B.Cu") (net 20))
 (segment (start 53.125 65.875) (end 52.05 66.95) (width 0.2) (layer "B.Cu") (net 20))
 (segment (start 44.275 62.25) (end 41.75 59.725) (width 0.2) (layer "B.Cu") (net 20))
 (segment (start 30.415 55.6) (end 30.625 55.81) (width 0.2) (layer "B.Cu") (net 20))
 (segment (start 41.75 59.725) (end 31.275 59.725) (width 0.2) (layer "B.Cu") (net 20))
 (segment (start 31.275 59.725) (end 31.1 59.55) (width 0.2) (layer "B.Cu") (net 20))
 (segment (start 48.577241 47.548139) (end 50.123139 47.548139) (width 0.2) (layer "B.Cu") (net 20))
 (segment (start 44.275 65.375) (end 44.275 62.25) (width 0.2) (layer "B.Cu") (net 20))
 (segment (start 53.125 50.55) (end 53.125 65.875) (width 0.2) (layer "B.Cu") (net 20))
 (segment (start 50.123139 47.548139) (end 53.125 50.55) (width 0.2) (layer "B.Cu") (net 20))
 (segment (start 28.775 56.4) (end 29.575 55.6) (width 0.2) (layer "B.Cu") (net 20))
 (segment (start 28.775 59.25) (end 28.775 56.4) (width 0.2) (layer "B.Cu") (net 20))
 (segment (start 45.85 66.95) (end 44.275 65.375) (width 0.2) (layer "B.Cu") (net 20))
 (segment (start 29.075 59.55) (end 28.775 59.25) (width 0.2) (layer "B.Cu") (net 20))
 (segment (start 34.275 48.725) (end 32.425 46.875) (width 0.2) (layer "B.Cu") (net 16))
 (segment (start 47.81 42.215) (end 41.3 48.725) (width 0.2) (layer "B.Cu") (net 16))
 (segment (start 41.3 48.725) (end 34.275 48.725) (width 0.2) (layer "B.Cu") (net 16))
 (segment (start 32.425 46.875) (end 32.425 46.1) (width 0.2) (layer "B.Cu") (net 16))
 (segment (start 31.975 45.65) (end 30.625 45.65) (width 0.2) (layer "B.Cu") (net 16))
 (segment (start 32.425 46.1) (end 31.975 45.65) (width 0.2) (layer "B.Cu") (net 16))
 (segment (start 48.615 42.215) (end 47.81 42.215) (width 0.2) (layer "B.Cu") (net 16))
 (segment (start 34.711442 81.21) (end 30.625 81.21) (width 0.4) (layer "F.Cu") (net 3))
 (segment (start 34.712978 81.208464) (end 34.711442 81.21) (width 0.4) (layer "F.Cu") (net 3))
 (via (at 39.45 79.675) (size 0.8) (drill 0.4) (layers "F.Cu" "B.Cu") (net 3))
 (segment (start 36.905927 82.378835) (end 36.905927 82.219073) (width 0.2) (layer "B.Cu") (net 3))
 (segment (start 36.905927 82.219073) (end 39.45 79.675) (width 0.2) (layer "B.Cu") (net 3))
 (segment (start 30.625 53.27) (end 26.845 53.27) (width 0.2) (layer "F.Cu") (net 19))
 (segment (start 42.3 27.875) (end 44.63 30.205) (width 0.2) (layer "F.Cu") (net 19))
 (segment (start 44.63 30.205) (end 44.63 32.280833) (width 0.2) (layer "F.Cu") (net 19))
 (segment (start 26.2 29.25) (end 27.575 27.875) (width 0.2) (layer "F.Cu") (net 19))
 (segment (start 27.575 27.875) (end 42.3 27.875) (width 0.2) (layer "F.Cu") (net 19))
 (segment (start 26.845 53.27) (end 26.2 52.625) (width 0.2) (layer "F.Cu") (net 19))
 (segment (start 26.2 52.625) (end 26.2 29.25) (width 0.2) (layer "F.Cu") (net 19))
 (segment (start 30.625 71.05) (end 34.099167 71.05) (width 0.25) (layer "F.Cu") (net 11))
 (segment (start 34.099167 71.05) (end 34.135 71.085833) (width 0.25) (layer "F.Cu") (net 11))
 (segment (start 33.425 56.725) (end 32.4 57.75) (width 0.2) (layer "F.Cu") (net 12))
 (segment (start 39.825 55.298082) (end 39.825 56.5) (width 0.2) (layer "F.Cu") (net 12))
 (segment (start 31.71 60.89) (end 30.625 60.89) (width 0.2) (layer "F.Cu") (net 12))
 (segment (start 42.614167 53.615) (end 41.508082 53.615) (width 0.2) (layer "F.Cu") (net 12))
 (segment (start 39.825 56.5) (end 39.6 56.725) (width 0.2) (layer "F.Cu") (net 12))
 (segment (start 39.6 56.725) (end 33.425 56.725) (width 0.2) (layer "F.Cu") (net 12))
 (segment (start 32.4 60.2) (end 31.71 60.89) (width 0.2) (layer "F.Cu") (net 12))
 (segment (start 41.508082 53.615) (end 39.825 55.298082) (width 0.2) (layer "F.Cu") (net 12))
 (segment (start 32.4 57.75) (end 32.4 60.2) (width 0.2) (layer "F.Cu") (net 12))
 (segment (start 45.375 86.8) (end 34.75 86.8) (width 0.2) (layer "B.Cu") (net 41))
 (segment (start 33.675 75.895898) (end 35.003139 74.567759) (width 0.2) (layer "B.Cu") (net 41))
 (segment (start 34.75 86.8) (end 33.675 85.725) (width 0.2) (layer "B.Cu") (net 41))
 (segment (start 33.675 85.725) (end 33.675 75.895898) (width 0.2) (layer "B.Cu") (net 41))
 (segment (start 47.457022 84.717978) (end 45.375 86.8) (width 0.2) (layer "B.Cu") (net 41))
 (segment (start 47.457022 82.362631) (end 47.457022 84.717978) (width 0.2) (layer "B.Cu") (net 41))
 (segment (start 53.125 60.53) (end 56.025 63.43) (width 0.2) (layer "F.Cu") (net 8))
 (segment (start 50.96 60.53) (end 53.125 60.53) (width 0.2) (layer "F.Cu") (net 8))
 (segment (start 53.155927 49.844073) (end 50.881165 49.844073) (width 0.2) (layer "F.Cu") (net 6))
 (segment (start 54.6 48.4) (end 53.155927 49.844073) (width 0.2) (layer "F.Cu") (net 6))
 (segment (start 54.6 38.675) (end 54.6 48.4) (width 0.2) (layer "F.Cu") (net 6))
 (segment (start 55.245 38.03) (end 54.6 38.675) (width 0.2) (layer "F.Cu") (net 6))
 (segment (start 56.025 38.03) (end 55.245 38.03) (width 0.2) (layer "F.Cu") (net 6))
 (segment (start 46.225 52.65) (end 46.225 66.505) (width 0.2) (layer "F.Cu") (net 10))
 (segment (start 52.02 72.3) (end 51.06 71.34) (width 0.2) (layer "F.Cu") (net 10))
 (segment (start 46.225 66.505) (end 51.06 71.34) (width 0.2) (layer "F.Cu") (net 10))
 (segment (start 46.35 52.525) (end 46.225 52.65) (width 0.2) (layer "F.Cu") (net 10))
 (segment (start 56.025 53.27) (end 55.28 52.525) (width 0.2) (layer "F.Cu") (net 10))
 (segment (start 55.28 52.525) (end 46.35 52.525) (width 0.2) (layer "F.Cu") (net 10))
 (segment (start 51.53538 55.81) (end 50.922241 55.196861) (width 0.2) (layer "F.Cu") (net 7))
 (segment (start 56.025 55.81) (end 51.53538 55.81) (width 0.2) (layer "F.Cu") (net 7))
 (segment (start 46.9 63.525) (end 49.315 65.94) (width 0.2) (layer "F.Cu") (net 9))
 (segment (start 56.025 60.89) (end 54.275 59.14) (width 0.2) (layer "F.Cu") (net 9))
 (segment (start 54.275 59.14) (end 54.275 58) (width 0.2) (layer "F.Cu") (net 9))
 (segment (start 54.275 58) (end 54.1 57.825) (width 0.2) (layer "F.Cu") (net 9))
 (segment (start 49.315 65.94) (end 51.06 65.94) (width 0.2) (layer "F.Cu") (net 9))
 (segment (start 54.1 57.825) (end 47.4 57.825) (width 0.2) (layer "F.Cu") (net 9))
 (segment (start 47.4 57.825) (end 46.9 58.325) (width 0.2) (layer "F.Cu") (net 9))
 (segment (start 46.9 58.325) (end 46.9 63.525) (width 0.2) (layer "F.Cu") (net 9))
 (segment (start 58.9 49.558862) (end 58.9 29.325) (width 0.2) (layer "F.Cu") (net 35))
 (segment (start 36.512369 36.887631) (end 36.512369 38.137978) (width 0.2) (layer "F.Cu") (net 35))
 (segment (start 56.625 27.05) (end 50.7 27.05) (width 0.2) (layer "F.Cu") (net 35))
 (segment (start 50.7 27.05) (end 47.325 30.425) (width 0.2) (layer "F.Cu") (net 35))
 (segment (start 47.325 30.425) (end 47.325 34.525) (width 0.2) (layer "F.Cu") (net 35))
 (segment (start 58.925 49.583862) (end 58.9 49.558862) (width 0.2) (layer "F.Cu") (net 35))
 (segment (start 46.925 34.925) (end 38.475 34.925) (width 0.2) (layer "F.Cu") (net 35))
 (segment (start 56.025 71.05) (end 58.225 71.05) (width 0.2) (layer "F.Cu") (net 35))
 (segment (start 47.325 34.525) (end 46.925 34.925) (width 0.2) (layer "F.Cu") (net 35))
 (segment (start 58.225 71.05) (end 58.925 70.35) (width 0.2) (layer "F.Cu") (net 35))
 (segment (start 58.9 29.325) (end 56.625 27.05) (width 0.2) (layer "F.Cu") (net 35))
 (segment (start 38.475 34.925) (end 36.512369 36.887631) (width 0.2) (layer "F.Cu") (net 35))
 (segment (start 58.925 70.35) (end 58.925 49.583862) (width 0.2) (layer "F.Cu") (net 35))
 (segment (start 32.8 44.7) (end 34.045 43.455) (width 0.2) (layer "F.Cu") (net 36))
 (segment (start 34.045 43.455) (end 36.515 43.455) (width 0.2) (layer "F.Cu") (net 36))
 (segment (start 23.2 26.85) (end 23.2 53.6) (width 0.2) (layer "F.Cu") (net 36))
 (segment (start 24.35 25.7) (end 23.2 26.85) (width 0.2) (layer "F.Cu") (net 36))
 (segment (start 26.65 57.05) (end 31.55 57.05) (width 0.2) (layer "F.Cu") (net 36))
 (segment (start 57.775 25.7) (end 24.35 25.7) (width 0.2) (layer "F.Cu") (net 36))
 (segment (start 56.025 73.59) (end 57.96 73.59) (width 0.2) (layer "F.Cu") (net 36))
 (segment (start 59.925 71.625) (end 59.925 27.85) (width 0.2) (layer "F.Cu") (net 36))
 (segment (start 23.2 53.6) (end 26.65 57.05) (width 0.2) (layer "F.Cu") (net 36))
 (segment (start 59.925 27.85) (end 57.775 25.7) (width 0.2) (layer "F.Cu") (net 36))
 (segment (start 32.8 55.8) (end 32.8 44.7) (width 0.2) (layer "F.Cu") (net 36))
 (segment (start 57.96 73.59) (end 59.925 71.625) (width 0.2) (layer "F.Cu") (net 36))
 (segment (start 31.55 57.05) (end 32.8 55.8) (width 0.2) (layer "F.Cu") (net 36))
 (segment (start 50.92 81.585833) (end 50.92 87.03) (width 0.2) (layer "F.Cu") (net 22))
 (segment (start 50.075 87.875) (end 29.5 87.875) (width 0.2) (layer "F.Cu") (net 22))
 (segment (start 50.92 87.03) (end 50.075 87.875) (width 0.2) (layer "F.Cu") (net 22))
 (segment (start 26.5 67.555) (end 30.625 63.43) (width 0.2) (layer "F.Cu") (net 22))
 (segment (start 29.5 87.875) (end 26.5 84.875) (width 0.2) (layer "F.Cu") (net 22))
 (segment (start 26.5 84.875) (end 26.5 67.555) (width 0.2) (layer "F.Cu") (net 22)))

